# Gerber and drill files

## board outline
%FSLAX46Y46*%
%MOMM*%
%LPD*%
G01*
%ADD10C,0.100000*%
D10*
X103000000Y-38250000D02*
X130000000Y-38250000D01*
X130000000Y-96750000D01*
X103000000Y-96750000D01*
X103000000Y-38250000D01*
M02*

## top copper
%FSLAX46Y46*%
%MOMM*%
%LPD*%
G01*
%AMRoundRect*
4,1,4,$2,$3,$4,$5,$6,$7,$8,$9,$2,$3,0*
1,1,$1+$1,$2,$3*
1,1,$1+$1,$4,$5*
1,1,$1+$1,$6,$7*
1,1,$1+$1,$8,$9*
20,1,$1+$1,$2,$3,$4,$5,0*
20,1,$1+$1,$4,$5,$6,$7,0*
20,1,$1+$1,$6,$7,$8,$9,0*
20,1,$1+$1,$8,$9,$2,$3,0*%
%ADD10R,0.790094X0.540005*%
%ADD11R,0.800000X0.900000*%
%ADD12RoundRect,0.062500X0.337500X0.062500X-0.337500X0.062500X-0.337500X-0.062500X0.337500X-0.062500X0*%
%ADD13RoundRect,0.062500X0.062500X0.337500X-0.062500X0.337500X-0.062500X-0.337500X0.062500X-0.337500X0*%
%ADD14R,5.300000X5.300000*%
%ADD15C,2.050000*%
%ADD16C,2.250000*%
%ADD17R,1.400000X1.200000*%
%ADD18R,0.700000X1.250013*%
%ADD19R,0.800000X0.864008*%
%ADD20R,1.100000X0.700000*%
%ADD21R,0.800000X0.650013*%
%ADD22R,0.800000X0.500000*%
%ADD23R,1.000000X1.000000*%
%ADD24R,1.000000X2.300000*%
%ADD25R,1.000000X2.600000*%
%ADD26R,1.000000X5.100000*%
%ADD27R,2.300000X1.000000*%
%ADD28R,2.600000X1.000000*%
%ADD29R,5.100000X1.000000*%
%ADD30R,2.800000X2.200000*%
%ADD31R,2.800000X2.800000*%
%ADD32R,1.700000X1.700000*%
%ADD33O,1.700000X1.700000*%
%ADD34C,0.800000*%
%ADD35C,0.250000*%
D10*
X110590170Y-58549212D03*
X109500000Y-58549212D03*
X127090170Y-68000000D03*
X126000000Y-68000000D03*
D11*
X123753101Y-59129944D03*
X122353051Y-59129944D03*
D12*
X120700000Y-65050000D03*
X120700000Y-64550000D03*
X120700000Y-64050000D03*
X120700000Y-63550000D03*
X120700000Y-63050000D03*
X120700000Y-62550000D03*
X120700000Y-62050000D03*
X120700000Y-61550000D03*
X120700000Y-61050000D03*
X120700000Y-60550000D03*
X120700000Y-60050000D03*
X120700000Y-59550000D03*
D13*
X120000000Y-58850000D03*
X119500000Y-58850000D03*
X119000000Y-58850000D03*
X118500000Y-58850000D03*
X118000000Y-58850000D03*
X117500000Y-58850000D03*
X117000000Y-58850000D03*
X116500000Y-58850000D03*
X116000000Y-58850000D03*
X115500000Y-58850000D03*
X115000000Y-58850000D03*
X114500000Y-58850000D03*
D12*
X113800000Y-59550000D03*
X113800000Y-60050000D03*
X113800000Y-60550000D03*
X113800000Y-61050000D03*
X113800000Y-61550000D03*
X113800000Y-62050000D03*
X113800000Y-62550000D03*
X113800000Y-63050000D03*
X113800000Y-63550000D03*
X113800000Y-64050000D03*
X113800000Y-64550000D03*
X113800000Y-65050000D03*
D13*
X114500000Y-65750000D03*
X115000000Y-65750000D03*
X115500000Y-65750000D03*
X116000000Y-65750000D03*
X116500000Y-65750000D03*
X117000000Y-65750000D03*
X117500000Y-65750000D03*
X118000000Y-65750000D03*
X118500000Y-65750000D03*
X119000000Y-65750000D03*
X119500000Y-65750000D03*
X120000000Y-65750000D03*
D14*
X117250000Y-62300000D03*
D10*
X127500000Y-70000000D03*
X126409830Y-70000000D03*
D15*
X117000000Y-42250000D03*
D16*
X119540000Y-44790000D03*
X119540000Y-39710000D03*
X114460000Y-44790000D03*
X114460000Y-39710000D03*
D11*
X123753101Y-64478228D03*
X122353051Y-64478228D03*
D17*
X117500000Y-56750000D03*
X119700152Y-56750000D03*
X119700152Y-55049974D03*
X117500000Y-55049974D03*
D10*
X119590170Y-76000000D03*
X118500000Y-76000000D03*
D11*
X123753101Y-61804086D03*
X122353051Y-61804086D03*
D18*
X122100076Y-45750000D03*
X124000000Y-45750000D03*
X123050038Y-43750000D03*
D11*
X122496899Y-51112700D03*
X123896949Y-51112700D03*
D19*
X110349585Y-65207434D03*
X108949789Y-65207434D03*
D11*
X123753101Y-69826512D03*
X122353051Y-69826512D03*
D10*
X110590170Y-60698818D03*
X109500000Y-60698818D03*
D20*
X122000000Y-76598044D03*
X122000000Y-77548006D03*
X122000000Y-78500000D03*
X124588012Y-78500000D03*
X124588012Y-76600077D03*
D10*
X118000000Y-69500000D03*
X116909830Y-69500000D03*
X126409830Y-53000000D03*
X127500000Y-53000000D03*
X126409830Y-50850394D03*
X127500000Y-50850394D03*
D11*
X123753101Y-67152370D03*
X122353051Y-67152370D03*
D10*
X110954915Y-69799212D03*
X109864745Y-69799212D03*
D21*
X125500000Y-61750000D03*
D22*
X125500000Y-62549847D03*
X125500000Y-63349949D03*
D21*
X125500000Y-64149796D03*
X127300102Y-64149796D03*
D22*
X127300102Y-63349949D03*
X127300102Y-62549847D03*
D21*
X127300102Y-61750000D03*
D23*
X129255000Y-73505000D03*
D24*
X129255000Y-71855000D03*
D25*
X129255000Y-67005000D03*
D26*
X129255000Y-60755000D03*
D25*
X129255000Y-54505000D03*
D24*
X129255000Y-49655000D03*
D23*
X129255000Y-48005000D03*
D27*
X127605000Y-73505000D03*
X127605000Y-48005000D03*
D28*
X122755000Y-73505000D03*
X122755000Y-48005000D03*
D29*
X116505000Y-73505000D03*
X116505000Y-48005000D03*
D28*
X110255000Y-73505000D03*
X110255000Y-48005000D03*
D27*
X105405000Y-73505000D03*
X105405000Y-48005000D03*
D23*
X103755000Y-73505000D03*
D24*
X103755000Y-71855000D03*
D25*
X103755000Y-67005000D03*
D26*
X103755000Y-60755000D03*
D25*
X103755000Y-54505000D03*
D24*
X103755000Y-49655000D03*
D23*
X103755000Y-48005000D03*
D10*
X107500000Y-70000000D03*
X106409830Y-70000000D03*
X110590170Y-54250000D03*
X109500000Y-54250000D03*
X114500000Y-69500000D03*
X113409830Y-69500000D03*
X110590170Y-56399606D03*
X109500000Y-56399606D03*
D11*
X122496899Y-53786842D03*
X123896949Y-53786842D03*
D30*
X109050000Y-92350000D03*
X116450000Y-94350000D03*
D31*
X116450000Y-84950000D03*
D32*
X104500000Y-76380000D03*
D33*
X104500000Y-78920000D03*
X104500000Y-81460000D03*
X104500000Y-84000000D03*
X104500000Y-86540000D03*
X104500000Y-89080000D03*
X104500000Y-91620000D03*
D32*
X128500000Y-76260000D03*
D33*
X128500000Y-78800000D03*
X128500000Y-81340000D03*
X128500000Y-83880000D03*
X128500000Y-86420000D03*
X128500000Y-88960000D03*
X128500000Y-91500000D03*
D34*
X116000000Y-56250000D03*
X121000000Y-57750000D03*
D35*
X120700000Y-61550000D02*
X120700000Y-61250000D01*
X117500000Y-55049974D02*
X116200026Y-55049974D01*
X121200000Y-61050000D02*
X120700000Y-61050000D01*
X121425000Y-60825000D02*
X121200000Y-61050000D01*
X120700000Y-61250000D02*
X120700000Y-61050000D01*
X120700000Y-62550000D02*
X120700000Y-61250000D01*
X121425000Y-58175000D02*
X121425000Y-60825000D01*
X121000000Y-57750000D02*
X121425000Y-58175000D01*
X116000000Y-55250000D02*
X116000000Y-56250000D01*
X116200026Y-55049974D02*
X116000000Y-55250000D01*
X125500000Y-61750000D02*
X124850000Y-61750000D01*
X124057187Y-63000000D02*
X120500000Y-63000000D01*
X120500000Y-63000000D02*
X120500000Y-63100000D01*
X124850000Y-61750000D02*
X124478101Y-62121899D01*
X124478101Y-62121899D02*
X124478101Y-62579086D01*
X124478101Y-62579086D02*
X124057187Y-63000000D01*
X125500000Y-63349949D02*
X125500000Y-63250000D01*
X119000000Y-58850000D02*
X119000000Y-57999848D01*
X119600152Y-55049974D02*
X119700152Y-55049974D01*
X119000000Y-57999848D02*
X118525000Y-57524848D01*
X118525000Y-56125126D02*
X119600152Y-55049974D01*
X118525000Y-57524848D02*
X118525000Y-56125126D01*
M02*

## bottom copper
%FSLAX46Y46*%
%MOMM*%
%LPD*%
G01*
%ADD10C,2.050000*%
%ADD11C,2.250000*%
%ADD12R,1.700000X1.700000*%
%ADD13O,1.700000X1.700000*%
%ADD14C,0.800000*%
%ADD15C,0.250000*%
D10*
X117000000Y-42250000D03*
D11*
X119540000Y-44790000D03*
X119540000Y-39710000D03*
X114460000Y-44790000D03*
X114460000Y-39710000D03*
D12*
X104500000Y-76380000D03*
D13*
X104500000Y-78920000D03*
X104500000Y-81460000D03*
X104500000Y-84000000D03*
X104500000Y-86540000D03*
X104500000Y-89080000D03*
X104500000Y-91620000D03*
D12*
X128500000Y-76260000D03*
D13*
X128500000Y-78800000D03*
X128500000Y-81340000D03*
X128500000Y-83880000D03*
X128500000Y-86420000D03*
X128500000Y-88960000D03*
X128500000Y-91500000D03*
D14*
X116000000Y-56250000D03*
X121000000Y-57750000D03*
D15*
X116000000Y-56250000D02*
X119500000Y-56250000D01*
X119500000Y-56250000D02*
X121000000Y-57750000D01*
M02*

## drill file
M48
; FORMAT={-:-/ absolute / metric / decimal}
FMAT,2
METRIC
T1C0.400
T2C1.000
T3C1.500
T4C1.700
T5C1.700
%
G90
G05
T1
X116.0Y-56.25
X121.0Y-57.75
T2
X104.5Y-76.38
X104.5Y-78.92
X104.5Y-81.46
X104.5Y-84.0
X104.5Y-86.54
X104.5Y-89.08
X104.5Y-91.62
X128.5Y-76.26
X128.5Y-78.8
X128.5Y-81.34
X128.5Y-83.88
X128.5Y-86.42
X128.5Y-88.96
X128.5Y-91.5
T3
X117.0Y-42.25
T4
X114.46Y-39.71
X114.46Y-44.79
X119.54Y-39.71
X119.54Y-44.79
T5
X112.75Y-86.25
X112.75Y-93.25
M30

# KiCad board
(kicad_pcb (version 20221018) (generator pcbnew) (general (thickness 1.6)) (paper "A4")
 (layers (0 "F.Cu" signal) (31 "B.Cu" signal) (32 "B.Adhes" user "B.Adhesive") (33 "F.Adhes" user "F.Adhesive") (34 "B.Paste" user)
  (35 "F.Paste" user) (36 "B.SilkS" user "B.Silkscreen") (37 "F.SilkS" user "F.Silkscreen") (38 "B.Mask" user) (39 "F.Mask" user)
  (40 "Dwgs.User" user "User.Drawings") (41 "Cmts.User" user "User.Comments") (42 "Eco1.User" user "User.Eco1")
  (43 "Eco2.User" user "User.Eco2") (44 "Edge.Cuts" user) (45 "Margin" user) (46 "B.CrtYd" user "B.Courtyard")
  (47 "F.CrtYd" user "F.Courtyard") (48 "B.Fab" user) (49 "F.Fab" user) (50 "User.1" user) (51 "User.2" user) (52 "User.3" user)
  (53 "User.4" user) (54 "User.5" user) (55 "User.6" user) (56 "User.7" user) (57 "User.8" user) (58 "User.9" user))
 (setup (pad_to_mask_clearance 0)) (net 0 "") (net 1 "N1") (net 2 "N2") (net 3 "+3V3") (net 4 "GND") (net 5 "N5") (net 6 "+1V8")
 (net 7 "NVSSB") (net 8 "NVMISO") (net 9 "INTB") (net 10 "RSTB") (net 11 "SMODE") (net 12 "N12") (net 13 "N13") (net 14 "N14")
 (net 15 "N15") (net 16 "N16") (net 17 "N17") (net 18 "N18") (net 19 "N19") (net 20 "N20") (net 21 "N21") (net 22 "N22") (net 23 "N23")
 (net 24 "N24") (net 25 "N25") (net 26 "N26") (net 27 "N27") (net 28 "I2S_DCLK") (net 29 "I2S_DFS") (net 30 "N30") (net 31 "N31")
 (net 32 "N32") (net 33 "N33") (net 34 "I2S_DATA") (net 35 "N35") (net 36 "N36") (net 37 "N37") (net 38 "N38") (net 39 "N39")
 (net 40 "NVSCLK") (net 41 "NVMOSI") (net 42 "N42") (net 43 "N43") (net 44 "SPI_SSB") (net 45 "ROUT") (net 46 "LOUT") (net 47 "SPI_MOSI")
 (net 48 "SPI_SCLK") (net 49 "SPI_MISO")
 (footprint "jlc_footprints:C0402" (layer "F.Cu") (at 110.045085 58.549212 180)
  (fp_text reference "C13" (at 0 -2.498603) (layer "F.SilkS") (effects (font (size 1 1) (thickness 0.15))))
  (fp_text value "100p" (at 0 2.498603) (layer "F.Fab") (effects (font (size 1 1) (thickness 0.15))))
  (pad "1" smd rect (at -0.545085 0 180) (size 0.790094 0.540005) (layers "F.Cu" "F.Paste" "F.Mask") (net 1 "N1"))
  (pad "2" smd rect (at 0.545085 0 180) (size 0.790094 0.540005) (layers "F.Cu" "F.Paste" "F.Mask") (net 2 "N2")))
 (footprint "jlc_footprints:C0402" (layer "F.Cu") (at 126.545085 68 180)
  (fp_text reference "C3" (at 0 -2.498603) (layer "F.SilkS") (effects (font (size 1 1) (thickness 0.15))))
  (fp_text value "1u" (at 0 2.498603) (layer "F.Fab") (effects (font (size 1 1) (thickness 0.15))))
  (pad "1" smd rect (at -0.545085 0 180) (size 0.790094 0.540005) (layers "F.Cu" "F.Paste" "F.Mask") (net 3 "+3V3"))
  (pad "2" smd rect (at 0.545085 0 180) (size 0.790094 0.540005) (layers "F.Cu" "F.Paste" "F.Mask") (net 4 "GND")))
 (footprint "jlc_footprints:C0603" (layer "F.Cu") (at 123.053076 59.129944 180)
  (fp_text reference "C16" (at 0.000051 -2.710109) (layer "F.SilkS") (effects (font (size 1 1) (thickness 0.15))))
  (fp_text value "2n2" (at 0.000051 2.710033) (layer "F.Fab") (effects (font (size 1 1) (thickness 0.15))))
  (pad "1" smd rect (at -0.700025 0 180) (size 0.8 0.9) (layers "F.Cu" "F.Paste" "F.Mask") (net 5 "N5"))
  (pad "2" smd rect (at 0.700025 0 180) (size 0.8 0.9) (layers "F.Cu" "F.Paste" "F.Mask") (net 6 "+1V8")))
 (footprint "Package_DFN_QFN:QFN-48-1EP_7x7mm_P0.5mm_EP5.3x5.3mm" (layer "F.Cu") (at 117.25 62.3 180)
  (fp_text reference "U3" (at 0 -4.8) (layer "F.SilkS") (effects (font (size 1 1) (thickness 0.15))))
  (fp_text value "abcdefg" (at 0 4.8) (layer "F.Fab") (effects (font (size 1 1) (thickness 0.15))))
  (pad "" smd roundrect (at -1.98 -1.98 180) (size 1.07 1.07) (layers "F.Paste") (roundrect_rratio 0.2336448598))
  (pad "" smd roundrect (at -1.98 -0.66 180) (size 1.07 1.07) (layers "F.Paste") (roundrect_rratio 0.2336448598))
  (pad "" smd roundrect (at -1.98 0.66 180) (size 1.07 1.07) (layers "F.Paste") (roundrect_rratio 0.2336448598))
  (pad "" smd roundrect (at -1.98 1.98 180) (size 1.07 1.07) (layers "F.Paste") (roundrect_rratio 0.2336448598))
  (pad "" smd roundrect (at -0.66 -1.98 180) (size 1.07 1.07) (layers "F.Paste") (roundrect_rratio 0.2336448598))
  (pad "" smd roundrect (at -0.66 -0.66 180) (size 1.07 1.07) (layers "F.Paste") (roundrect_rratio 0.2336448598))
  (pad "" smd roundrect (at -0.66 0.66 180) (size 1.07 1.07) (layers "F.Paste") (roundrect_rratio 0.2336448598))
  (pad "" smd roundrect (at -0.66 1.98 180) (size 1.07 1.07) (layers "F.Paste") (roundrect_rratio 0.2336448598))
  (pad "" smd roundrect (at 0.66 -1.98 180) (size 1.07 1.07) (layers "F.Paste") (roundrect_rratio 0.2336448598))
  (pad "" smd roundrect (at 0.66 -0.66 180) (size 1.07 1.07) (layers "F.Paste") (roundrect_rratio 0.2336448598))
  (pad "" smd roundrect (at 0.66 0.66 180) (size 1.07 1.07) (layers "F.Paste") (roundrect_rratio 0.2336448598))
  (pad "" smd roundrect (at 0.66 1.98 180) (size 1.07 1.07) (layers "F.Paste") (roundrect_rratio 0.2336448598))
  (pad "" smd roundrect (at 1.98 -1.98 180) (size 1.07 1.07) (layers "F.Paste") (roundrect_rratio 0.2336448598))
  (pad "" smd roundrect (at 1.98 -0.66 180) (size 1.07 1.07) (layers "F.Paste") (roundrect_rratio 0.2336448598))
  (pad "" smd roundrect (at 1.98 0.66 180) (size 1.07 1.07) (layers "F.Paste") (roundrect_rratio 0.2336448598))
  (pad "" smd roundrect (at 1.98 1.98 180) (size 1.07 1.07) (layers "F.Paste") (roundrect_rratio 0.2336448598))
  (pad "1" smd roundrect (at -3.45 -2.75 180) (size 0.8 0.25) (layers "F.Cu" "F.Paste" "F.Mask") (roundrect_rratio 0.25) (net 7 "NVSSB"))
  (pad "2" smd roundrect (at -3.45 -2.25 180) (size 0.8 0.25) (layers "F.Cu" "F.Paste" "F.Mask") (roundrect_rratio 0.25) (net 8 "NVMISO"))
  (pad "3" smd roundrect (at -3.45 -1.75 180) (size 0.8 0.25) (layers "F.Cu" "F.Paste" "F.Mask") (roundrect_rratio 0.25) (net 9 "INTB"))
  (pad "4" smd roundrect (at -3.45 -1.25 180) (size 0.8 0.25) (layers "F.Cu" "F.Paste" "F.Mask") (roundrect_rratio 0.25) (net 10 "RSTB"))
  (pad "5" smd roundrect (at -3.45 -0.75 180) (size 0.8 0.25) (layers "F.Cu" "F.Paste" "F.Mask") (roundrect_rratio 0.25) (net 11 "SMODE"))
  (pad "6" smd roundrect (at -3.45 -0.25 180) (size 0.8 0.25) (layers "F.Cu" "F.Paste" "F.Mask") (roundrect_rratio 0.25) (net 4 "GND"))
  (pad "7" smd roundrect (at -3.45 0.25 180) (size 0.8 0.25) (layers "F.Cu" "F.Paste" "F.Mask") (roundrect_rratio 0.25) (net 4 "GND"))
  (pad "8" smd roundrect (at -3.45 0.75 180) (size 0.8 0.25) (layers "F.Cu" "F.Paste" "F.Mask") (roundrect_rratio 0.25) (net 4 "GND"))
  (pad "9" smd roundrect (at -3.45 1.25 180) (size 0.8 0.25) (layers "F.Cu" "F.Paste" "F.Mask") (roundrect_rratio 0.25) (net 4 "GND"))
  (pad "10" smd roundrect (at -3.45 1.75 180) (size 0.8 0.25) (layers "F.Cu" "F.Paste" "F.Mask") (roundrect_rratio 0.25) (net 2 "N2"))
  (pad "11" smd roundrect (at -3.45 2.25 180) (size 0.8 0.25) (layers "F.Cu" "F.Paste" "F.Mask") (roundrect_rratio 0.25) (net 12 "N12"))
  (pad "12" smd roundrect (at -3.45 2.75 180) (size 0.8 0.25) (layers "F.Cu" "F.Paste" "F.Mask") (roundrect_rratio 0.25) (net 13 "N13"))
  (pad "13" smd roundrect (at -2.75 3.45 180) (size 0.25 0.8) (layers "F.Cu" "F.Paste" "F.Mask") (roundrect_rratio 0.25) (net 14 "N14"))
  (pad "14" smd roundrect (at -2.25 3.45 180) (size 0.25 0.8) (layers "F.Cu" "F.Paste" "F.Mask") (roundrect_rratio 0.25) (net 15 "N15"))
  (pad "15" smd roundrect (at -1.75 3.45 180) (size 0.25 0.8) (layers "F.Cu" "F.Paste" "F.Mask") (roundrect_rratio 0.25) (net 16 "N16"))
  (pad "16" smd roundrect (at -1.25 3.45 180) (size 0.25 0.8) (layers "F.Cu" "F.Paste" "F.Mask") (roundrect_rratio 0.25) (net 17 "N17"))
  (pad "17" smd roundrect (at -0.75 3.45 180) (size 0.25 0.8) (layers "F.Cu" "F.Paste" "F.Mask") (roundrect_rratio 0.25) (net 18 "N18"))
  (pad "18" smd roundrect (at -0.25 3.45 180) (size 0.25 0.8) (layers "F.Cu" "F.Paste" "F.Mask") (roundrect_rratio 0.25) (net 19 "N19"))
  (pad "19" smd roundrect (at 0.25 3.45 180) (size 0.25 0.8) (layers "F.Cu" "F.Paste" "F.Mask") (roundrect_rratio 0.25) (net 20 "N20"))
  (pad "20" smd roundrect (at 0.75 3.45 180) (size 0.25 0.8) (layers "F.Cu" "F.Paste" "F.Mask") (roundrect_rratio 0.25) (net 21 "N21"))
  (pad "21" smd roundrect (at 1.25 3.45 180) (size 0.25 0.8) (layers "F.Cu" "F.Paste" "F.Mask") (roundrect_rratio 0.25) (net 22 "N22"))
  (pad "22" smd roundrect (at 1.75 3.45 180) (size 0.25 0.8) (layers "F.Cu" "F.Paste" "F.Mask") (roundrect_rratio 0.25) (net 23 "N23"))
  (pad "23" smd roundrect (at 2.25 3.45 180) (size 0.25 0.8) (layers "F.Cu" "F.Paste" "F.Mask") (roundrect_rratio 0.25) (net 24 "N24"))
  (pad "24" smd roundrect (at 2.75 3.45 180) (size 0.25 0.8) (layers "F.Cu" "F.Paste" "F.Mask") (roundrect_rratio 0.25) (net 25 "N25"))
  (pad "25" smd roundrect (at 3.45 2.75 180) (size 0.8 0.25) (layers "F.Cu" "F.Paste" "F.Mask") (roundrect_rratio 0.25) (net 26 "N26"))
  (pad "26" smd roundrect (at 3.45 2.25 180) (size 0.8 0.25) (layers "F.Cu" "F.Paste" "F.Mask") (roundrect_rratio 0.25) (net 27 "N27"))
  (pad "27" smd roundrect (at 3.45 1.75 180) (size 0.8 0.25) (layers "F.Cu" "F.Paste" "F.Mask") (roundrect_rratio 0.25) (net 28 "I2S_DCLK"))
  (pad "28" smd roundrect (at 3.45 1.25 180) (size 0.8 0.25) (layers "F.Cu" "F.Paste" "F.Mask") (roundrect_rratio 0.25) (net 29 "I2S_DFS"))
  (pad "29" smd roundrect (at 3.45 0.75 180) (size 0.8 0.25) (layers "F.Cu" "F.Paste" "F.Mask") (roundrect_rratio 0.25) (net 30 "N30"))
  (pad "30" smd roundrect (at 3.45 0.25 180) (size 0.8 0.25) (layers "F.Cu" "F.Paste" "F.Mask") (roundrect_rratio 0.25) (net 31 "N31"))
  (pad "31" smd roundrect (at 3.45 -0.25 180) (size 0.8 0.25) (layers "F.Cu" "F.Paste" "F.Mask") (roundrect_rratio 0.25) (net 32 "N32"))
  (pad "32" smd roundrect (at 3.45 -0.75 180) (size 0.8 0.25) (layers "F.Cu" "F.Paste" "F.Mask") (roundrect_rratio 0.25) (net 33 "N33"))
  (pad "33" smd roundrect (at 3.45 -1.25 180) (size 0.8 0.25) (layers "F.Cu" "F.Paste" "F.Mask") (roundrect_rratio 0.25) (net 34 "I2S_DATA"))
  (pad "34" smd roundrect (at 3.45 -1.75 180) (size 0.8 0.25) (layers "F.Cu" "F.Paste" "F.Mask") (roundrect_rratio 0.25) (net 3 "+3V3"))
  (pad "35" smd roundrect (at 3.45 -2.25 180) (size 0.8 0.25) (layers "F.Cu" "F.Paste" "F.Mask") (roundrect_rratio 0.25) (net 6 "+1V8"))
  (pad "36" smd roundrect (at 3.45 -2.75 180) (size 0.8 0.25) (layers "F.Cu" "F.Paste" "F.Mask") (roundrect_rratio 0.25) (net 5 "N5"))
  (pad "37" smd roundrect (at 2.75 -3.45 180) (size 0.25 0.8) (layers "F.Cu" "F.Paste" "F.Mask") (roundrect_rratio 0.25) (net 6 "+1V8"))
  (pad "38" smd roundrect (at 2.25 -3.45 180) (size 0.25 0.8) (layers "F.Cu" "F.Paste" "F.Mask") (roundrect_rratio 0.25) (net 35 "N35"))
  (pad "39" smd roundrect (at 1.75 -3.45 180) (size 0.25 0.8) (layers "F.Cu" "F.Paste" "F.Mask") (roundrect_rratio 0.25) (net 4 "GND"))
  (pad "40" smd roundrect (at 1.25 -3.45 180) (size 0.25 0.8) (layers "F.Cu" "F.Paste" "F.Mask") (roundrect_rratio 0.25) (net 4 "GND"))
  (pad "41" smd roundrect (at 0.75 -3.45 180) (size 0.25 0.8) (layers "F.Cu" "F.Paste" "F.Mask") (roundrect_rratio 0.25) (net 4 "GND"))
  (pad "42" smd roundrect (at 0.25 -3.45 180) (size 0.25 0.8) (layers "F.Cu" "F.Paste" "F.Mask") (roundrect_rratio 0.25) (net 4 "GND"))
  (pad "43" smd roundrect (at -0.25 -3.45 180) (size 0.25 0.8) (layers "F.Cu" "F.Paste" "F.Mask") (roundrect_rratio 0.25) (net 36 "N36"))
  (pad "44" smd roundrect (at -0.75 -3.45 180) (size 0.25 0.8) (layers "F.Cu" "F.Paste" "F.Mask") (roundrect_rratio 0.25) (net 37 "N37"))
  (pad "45" smd roundrect (at -1.25 -3.45 180) (size 0.25 0.8) (layers "F.Cu" "F.Paste" "F.Mask") (roundrect_rratio 0.25) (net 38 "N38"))
  (pad "46" smd roundrect (at -1.75 -3.45 180) (size 0.25 0.8) (layers "F.Cu" "F.Paste" "F.Mask") (roundrect_rratio 0.25) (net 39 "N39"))
  (pad "47" smd roundrect (at -2.25 -3.45 180) (size 0.25 0.8) (layers "F.Cu" "F.Paste" "F.Mask") (roundrect_rratio 0.25) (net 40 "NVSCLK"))
  (pad "48" smd roundrect (at -2.75 -3.45 180) (size 0.25 0.8) (layers "F.Cu" "F.Paste" "F.Mask") (roundrect_rratio 0.25) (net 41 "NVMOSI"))
  (pad "49" smd rect (at 0 0 180) (size 5.3 5.3) (layers "F.Cu" "F.Mask")))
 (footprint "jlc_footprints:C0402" (layer "F.Cu") (at 126.954915 70 180)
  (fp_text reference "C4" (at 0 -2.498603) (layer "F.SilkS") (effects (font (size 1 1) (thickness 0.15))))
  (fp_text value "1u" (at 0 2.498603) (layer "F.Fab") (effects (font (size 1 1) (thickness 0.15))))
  (pad "1" smd rect (at -0.545085 0 180) (size 0.790094 0.540005) (layers "F.Cu" "F.Paste" "F.Mask") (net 6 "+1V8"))
  (pad "2" smd rect (at 0.545085 0 180) (size 0.790094 0.540005) (layers "F.Cu" "F.Paste" "F.Mask") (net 4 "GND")))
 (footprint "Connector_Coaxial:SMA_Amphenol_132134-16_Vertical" (layer "F.Cu") (at 117 42.25 180)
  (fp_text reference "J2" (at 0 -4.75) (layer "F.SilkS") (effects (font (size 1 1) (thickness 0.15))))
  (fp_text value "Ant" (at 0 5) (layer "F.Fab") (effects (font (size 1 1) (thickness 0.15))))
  (pad "1" thru_hole circle (at 0 0 180) (size 2.05 2.05) (drill 1.5) (layers "*.Cu" "*.Mask") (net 1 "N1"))
  (pad "2" thru_hole circle (at -2.54 -2.54 180) (size 2.25 2.25) (drill 1.7) (layers "*.Cu" "*.Mask") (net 4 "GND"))
  (pad "2" thru_hole circle (at -2.54 2.54 180) (size 2.25 2.25) (drill 1.7) (layers "*.Cu" "*.Mask") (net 4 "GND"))
  (pad "2" thru_hole circle (at 2.54 -2.54 180) (size 2.25 2.25) (drill 1.7) (layers "*.Cu" "*.Mask") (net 4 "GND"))
  (pad "2" thru_hole circle (at 2.54 2.54 180) (size 2.25 2.25) (drill 1.7) (layers "*.Cu" "*.Mask") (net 4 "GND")))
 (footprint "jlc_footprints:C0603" (layer "F.Cu") (at 123.053076 64.478228 180)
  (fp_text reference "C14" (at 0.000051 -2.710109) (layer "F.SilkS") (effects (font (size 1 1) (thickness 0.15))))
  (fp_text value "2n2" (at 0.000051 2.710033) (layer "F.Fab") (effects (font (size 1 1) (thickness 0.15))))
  (pad "1" smd rect (at -0.700025 0 180) (size 0.8 0.9) (layers "F.Cu" "F.Paste" "F.Mask") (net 14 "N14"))
  (pad "2" smd rect (at 0.700025 0 180) (size 0.8 0.9) (layers "F.Cu" "F.Paste" "F.Mask") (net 13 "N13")))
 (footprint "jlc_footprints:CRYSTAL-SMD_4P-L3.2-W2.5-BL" (layer "F.Cu") (at 118.600076 55.899987)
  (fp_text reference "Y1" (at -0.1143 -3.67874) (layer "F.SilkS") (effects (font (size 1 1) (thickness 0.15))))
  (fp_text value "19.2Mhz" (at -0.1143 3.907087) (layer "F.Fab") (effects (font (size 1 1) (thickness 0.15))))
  (pad "1" smd rect (at -1.100076 0.850013) (size 1.4 1.2) (layers "F.Cu" "F.Paste" "F.Mask") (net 17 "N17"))
  (pad "2" smd rect (at 1.100076 0.850013) (size 1.4 1.2) (layers "F.Cu" "F.Paste" "F.Mask") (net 4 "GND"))
  (pad "3" smd rect (at 1.100076 -0.850013) (size 1.4 1.2) (layers "F.Cu" "F.Paste" "F.Mask") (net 16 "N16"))
  (pad "4" smd rect (at -1.100076 -0.850013) (size 1.4 1.2) (layers "F.Cu" "F.Paste" "F.Mask") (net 4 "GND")))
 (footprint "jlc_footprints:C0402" (layer "F.Cu") (at 119.045085 76 180)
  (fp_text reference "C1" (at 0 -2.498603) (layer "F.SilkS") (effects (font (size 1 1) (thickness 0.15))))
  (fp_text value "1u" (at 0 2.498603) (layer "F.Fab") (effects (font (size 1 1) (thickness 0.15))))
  (pad "1" smd rect (at -0.545085 0 180) (size 0.790094 0.540005) (layers "F.Cu" "F.Paste" "F.Mask") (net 4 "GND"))
  (pad "2" smd rect (at 0.545085 0 180) (size 0.790094 0.540005) (layers "F.Cu" "F.Paste" "F.Mask") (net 18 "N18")))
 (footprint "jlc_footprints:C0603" (layer "F.Cu") (at 123.053076 61.804086 180)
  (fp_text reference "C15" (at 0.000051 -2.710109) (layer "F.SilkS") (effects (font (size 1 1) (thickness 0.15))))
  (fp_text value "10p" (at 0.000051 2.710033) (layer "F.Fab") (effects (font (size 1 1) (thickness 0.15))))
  (pad "1" smd rect (at -0.700025 0 180) (size 0.8 0.9) (layers "F.Cu" "F.Paste" "F.Mask") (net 14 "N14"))
  (pad "2" smd rect (at 0.700025 0 180) (size 0.8 0.9) (layers "F.Cu" "F.Paste" "F.Mask") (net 13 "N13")))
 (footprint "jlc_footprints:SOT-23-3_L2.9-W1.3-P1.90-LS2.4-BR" (layer "F.Cu") (at 123.050038 44.75 -90)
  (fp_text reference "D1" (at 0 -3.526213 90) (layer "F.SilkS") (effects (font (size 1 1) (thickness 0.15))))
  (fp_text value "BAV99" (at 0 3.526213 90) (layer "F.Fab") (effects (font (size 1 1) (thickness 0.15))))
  (pad "1" smd rect (at 1 0.949962 270) (size 1.250013 0.7) (layers "F.Cu" "F.Paste" "F.Mask") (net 4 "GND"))
  (pad "2" smd rect (at 1 -0.949962 270) (size 1.250013 0.7) (layers "F.Cu" "F.Paste" "F.Mask") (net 4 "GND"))
  (pad "3" smd rect (at -1 0 270) (size 1.250013 0.7) (layers "F.Cu" "F.Paste" "F.Mask") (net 1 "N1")))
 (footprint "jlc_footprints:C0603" (layer "F.Cu") (at 123.196924 51.1127)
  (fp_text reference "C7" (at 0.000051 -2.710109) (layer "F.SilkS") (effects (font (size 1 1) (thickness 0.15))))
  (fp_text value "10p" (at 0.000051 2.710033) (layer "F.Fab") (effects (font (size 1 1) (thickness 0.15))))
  (pad "1" smd rect (at -0.700025 0) (size 0.8 0.9) (layers "F.Cu" "F.Paste" "F.Mask") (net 4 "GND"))
  (pad "2" smd rect (at 0.700025 0) (size 0.8 0.9) (layers "F.Cu" "F.Paste" "F.Mask") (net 20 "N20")))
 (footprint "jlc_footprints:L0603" (layer "F.Cu") (at 109.649687 65.207434 180)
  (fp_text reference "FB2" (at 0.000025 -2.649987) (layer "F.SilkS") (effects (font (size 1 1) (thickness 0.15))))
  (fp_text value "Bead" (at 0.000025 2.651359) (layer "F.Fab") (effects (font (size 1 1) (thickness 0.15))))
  (pad "1" smd rect (at -0.699898 0) (size 0.8 0.864008) (layers "F.Cu" "F.Paste" "F.Mask") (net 6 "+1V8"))
  (pad "2" smd rect (at 0.699898 0) (size 0.8 0.864008) (layers "F.Cu" "F.Paste" "F.Mask") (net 13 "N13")))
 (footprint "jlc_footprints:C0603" (layer "F.Cu") (at 123.053076 69.826512 180)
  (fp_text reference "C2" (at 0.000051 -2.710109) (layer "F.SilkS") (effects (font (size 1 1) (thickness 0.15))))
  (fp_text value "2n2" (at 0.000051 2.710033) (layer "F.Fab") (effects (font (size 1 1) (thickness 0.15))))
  (pad "1" smd rect (at -0.700025 0 180) (size 0.8 0.9) (layers "F.Cu" "F.Paste" "F.Mask") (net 5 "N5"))
  (pad "2" smd rect (at 0.700025 0 180) (size 0.8 0.9) (layers "F.Cu" "F.Paste" "F.Mask") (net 3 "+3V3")))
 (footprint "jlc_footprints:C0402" (layer "F.Cu") (at 110.045085 60.698818 180)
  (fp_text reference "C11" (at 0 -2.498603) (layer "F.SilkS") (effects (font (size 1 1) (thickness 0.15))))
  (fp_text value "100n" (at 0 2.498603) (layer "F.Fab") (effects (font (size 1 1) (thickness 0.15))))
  (pad "1" smd rect (at -0.545085 0 180) (size 0.790094 0.540005) (layers "F.Cu" "F.Paste" "F.Mask") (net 14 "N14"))
  (pad "2" smd rect (at 0.545085 0 180) (size 0.790094 0.540005) (layers "F.Cu" "F.Paste" "F.Mask") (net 13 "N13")))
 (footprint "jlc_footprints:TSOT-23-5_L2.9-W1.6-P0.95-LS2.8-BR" (layer "F.Cu") (at 123.294006 77.549124 180)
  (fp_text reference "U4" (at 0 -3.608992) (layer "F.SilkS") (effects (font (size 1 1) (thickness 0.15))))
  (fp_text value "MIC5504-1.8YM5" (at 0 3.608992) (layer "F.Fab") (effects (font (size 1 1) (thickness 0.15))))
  (pad "1" smd rect (at 1.294006 0.95108 180) (size 1.1 0.7) (layers "F.Cu" "F.Paste" "F.Mask") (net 3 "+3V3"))
  (pad "2" smd rect (at 1.294006 0.001118 180) (size 1.1 0.7) (layers "F.Cu" "F.Paste" "F.Mask") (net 4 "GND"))
  (pad "3" smd rect (at 1.294006 -0.950876 180) (size 1.1 0.7) (layers "F.Cu" "F.Paste" "F.Mask") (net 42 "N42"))
  (pad "4" smd rect (at -1.294006 -0.950876) (size 1.1 0.7) (layers "F.Cu" "F.Paste" "F.Mask") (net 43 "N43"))
  (pad "5" smd rect (at -1.294006 0.949047) (size 1.1 0.7) (layers "F.Cu" "F.Paste" "F.Mask") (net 6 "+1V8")))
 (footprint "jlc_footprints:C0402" (layer "F.Cu") (at 117.454915 69.5 180)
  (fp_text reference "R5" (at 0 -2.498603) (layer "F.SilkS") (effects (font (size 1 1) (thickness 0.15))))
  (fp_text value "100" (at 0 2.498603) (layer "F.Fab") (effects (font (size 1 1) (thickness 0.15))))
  (pad "1" smd rect (at -0.545085 0 180) (size 0.790094 0.540005) (layers "F.Cu" "F.Paste" "F.Mask") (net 30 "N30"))
  (pad "2" smd rect (at 0.545085 0 180) (size 0.790094 0.540005) (layers "F.Cu" "F.Paste" "F.Mask") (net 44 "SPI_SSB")))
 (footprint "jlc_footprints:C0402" (layer "F.Cu") (at 126.954915 53)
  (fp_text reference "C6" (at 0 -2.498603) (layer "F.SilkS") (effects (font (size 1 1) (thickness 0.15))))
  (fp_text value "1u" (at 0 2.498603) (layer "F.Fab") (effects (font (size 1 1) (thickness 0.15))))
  (pad "1" smd rect (at -0.545085 0) (size 0.790094 0.540005) (layers "F.Cu" "F.Paste" "F.Mask") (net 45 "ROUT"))
  (pad "2" smd rect (at 0.545085 0) (size 0.790094 0.540005) (layers "F.Cu" "F.Paste" "F.Mask") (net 20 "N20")))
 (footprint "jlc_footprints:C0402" (layer "F.Cu") (at 126.954915 50.850394)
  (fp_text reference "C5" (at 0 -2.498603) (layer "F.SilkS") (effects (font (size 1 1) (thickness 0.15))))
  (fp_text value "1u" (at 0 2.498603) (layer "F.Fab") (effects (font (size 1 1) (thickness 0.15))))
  (pad "1" smd rect (at -0.545085 0) (size 0.790094 0.540005) (layers "F.Cu" "F.Paste" "F.Mask") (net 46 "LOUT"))
  (pad "2" smd rect (at 0.545085 0) (size 0.790094 0.540005) (layers "F.Cu" "F.Paste" "F.Mask") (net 19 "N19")))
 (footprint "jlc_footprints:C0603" (layer "F.Cu") (at 123.053076 67.15237 180)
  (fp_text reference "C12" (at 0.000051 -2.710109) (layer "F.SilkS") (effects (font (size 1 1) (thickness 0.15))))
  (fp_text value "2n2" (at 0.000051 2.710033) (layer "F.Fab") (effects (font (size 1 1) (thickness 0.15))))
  (pad "1" smd rect (at -0.700025 0 180) (size 0.8 0.9) (layers "F.Cu" "F.Paste" "F.Mask") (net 5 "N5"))
  (pad "2" smd rect (at 0.700025 0 180) (size 0.8 0.9) (layers "F.Cu" "F.Paste" "F.Mask") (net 6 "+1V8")))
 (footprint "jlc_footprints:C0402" (layer "F.Cu") (at 110.40983 69.799212 180)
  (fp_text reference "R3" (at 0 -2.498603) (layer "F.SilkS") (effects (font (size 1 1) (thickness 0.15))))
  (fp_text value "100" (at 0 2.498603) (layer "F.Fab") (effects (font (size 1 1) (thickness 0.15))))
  (pad "1" smd rect (at -0.545085 0 180) (size 0.790094 0.540005) (layers "F.Cu" "F.Paste" "F.Mask") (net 32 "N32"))
  (pad "2" smd rect (at 0.545085 0 180) (size 0.790094 0.540005) (layers "F.Cu" "F.Paste" "F.Mask") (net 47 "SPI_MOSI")))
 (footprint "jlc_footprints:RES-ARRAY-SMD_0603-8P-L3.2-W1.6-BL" (layer "F.Cu") (at 126.400051 62.949898 -90)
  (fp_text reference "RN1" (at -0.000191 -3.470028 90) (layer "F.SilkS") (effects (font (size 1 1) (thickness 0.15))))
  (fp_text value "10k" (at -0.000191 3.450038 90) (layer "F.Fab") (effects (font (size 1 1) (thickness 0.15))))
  (pad "1" smd rect (at -1.199898 0.900051 270) (size 0.650013 0.8) (layers "F.Cu" "F.Paste" "F.Mask") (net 11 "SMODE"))
  (pad "2" smd rect (at -0.400051 0.900051 270) (size 0.5 0.8) (layers "F.Cu" "F.Paste" "F.Mask") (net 10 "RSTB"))
  (pad "3" smd rect (at 0.400051 0.900051 270) (size 0.5 0.8) (layers "F.Cu" "F.Paste" "F.Mask") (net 9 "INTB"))
  (pad "4" smd rect (at 1.199898 0.900051 270) (size 0.650013 0.8) (layers "F.Cu" "F.Paste" "F.Mask") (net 3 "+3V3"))
  (pad "5" smd rect (at 1.199898 -0.900051 270) (size 0.650013 0.8) (layers "F.Cu" "F.Paste" "F.Mask") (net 42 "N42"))
  (pad "6" smd rect (at 0.400051 -0.900051 270) (size 0.5 0.8) (layers "F.Cu" "F.Paste" "F.Mask") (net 3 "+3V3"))
  (pad "7" smd rect (at -0.400051 -0.900051 270) (size 0.5 0.8) (layers "F.Cu" "F.Paste" "F.Mask") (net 3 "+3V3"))
  (pad "8" smd rect (at -1.199898 -0.900051 270) (size 0.650013 0.8) (layers "F.Cu" "F.Paste" "F.Mask") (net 4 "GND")))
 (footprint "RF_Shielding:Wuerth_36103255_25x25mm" (layer "F.Cu") (at 116.505 60.755 180)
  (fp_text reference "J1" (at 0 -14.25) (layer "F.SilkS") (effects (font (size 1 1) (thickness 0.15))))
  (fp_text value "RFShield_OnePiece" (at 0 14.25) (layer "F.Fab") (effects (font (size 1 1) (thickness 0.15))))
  (pad "1" smd rect (at -12.75 -12.75 180) (size 1 1) (layers "F.Cu" "F.Paste" "F.Mask") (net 4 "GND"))
  (pad "1" smd rect (at -12.75 -11.1 180) (size 1 2.3) (layers "F.Cu" "F.Paste" "F.Mask") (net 4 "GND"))
  (pad "1" smd rect (at -12.75 -6.25 180) (size 1 2.6) (layers "F.Cu" "F.Paste" "F.Mask") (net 4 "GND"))
  (pad "1" smd rect (at -12.75 0 180) (size 1 5.1) (layers "F.Cu" "F.Paste" "F.Mask") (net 4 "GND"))
  (pad "1" smd rect (at -12.75 6.25 180) (size 1 2.6) (layers "F.Cu" "F.Paste" "F.Mask") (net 4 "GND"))
  (pad "1" smd rect (at -12.75 11.1 180) (size 1 2.3) (layers "F.Cu" "F.Paste" "F.Mask") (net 4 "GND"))
  (pad "1" smd rect (at -12.75 12.75 180) (size 1 1) (layers "F.Cu" "F.Paste" "F.Mask") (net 4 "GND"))
  (pad "1" smd rect (at -11.1 -12.75 180) (size 2.3 1) (layers "F.Cu" "F.Paste" "F.Mask") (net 4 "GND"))
  (pad "1" smd rect (at -11.1 12.75 180) (size 2.3 1) (layers "F.Cu" "F.Paste" "F.Mask") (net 4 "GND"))
  (pad "1" smd rect (at -6.25 -12.75 180) (size 2.6 1) (layers "F.Cu" "F.Paste" "F.Mask") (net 4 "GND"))
  (pad "1" smd rect (at -6.25 12.75 180) (size 2.6 1) (layers "F.Cu" "F.Paste" "F.Mask") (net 4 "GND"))
  (pad "1" smd rect (at 0 -12.75 180) (size 5.1 1) (layers "F.Cu" "F.Paste" "F.Mask") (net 4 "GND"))
  (pad "1" smd rect (at 0 12.75 180) (size 5.1 1) (layers "F.Cu" "F.Paste" "F.Mask") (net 4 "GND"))
  (pad "1" smd rect (at 6.25 -12.75 180) (size 2.6 1) (layers "F.Cu" "F.Paste" "F.Mask") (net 4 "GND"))
  (pad "1" smd rect (at 6.25 12.75 180) (size 2.6 1) (layers "F.Cu" "F.Paste" "F.Mask") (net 4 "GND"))
  (pad "1" smd rect (at 11.1 -12.75 180) (size 2.3 1) (layers "F.Cu" "F.Paste" "F.Mask") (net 4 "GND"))
  (pad "1" smd rect (at 11.1 12.75 180) (size 2.3 1) (layers "F.Cu" "F.Paste" "F.Mask") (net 4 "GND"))
  (pad "1" smd rect (at 12.75 -12.75 180) (size 1 1) (layers "F.Cu" "F.Paste" "F.Mask") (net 4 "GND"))
  (pad "1" smd rect (at 12.75 -11.1 180) (size 1 2.3) (layers "F.Cu" "F.Paste" "F.Mask") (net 4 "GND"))
  (pad "1" smd rect (at 12.75 -6.25 180) (size 1 2.6) (layers "F.Cu" "F.Paste" "F.Mask") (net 4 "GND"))
  (pad "1" smd rect (at 12.75 0 180) (size 1 5.1) (layers "F.Cu" "F.Paste" "F.Mask") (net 4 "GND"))
  (pad "1" smd rect (at 12.75 6.25 180) (size 1 2.6) (layers "F.Cu" "F.Paste" "F.Mask") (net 4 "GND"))
  (pad "1" smd rect (at 12.75 11.1 180) (size 1 2.3) (layers "F.Cu" "F.Paste" "F.Mask") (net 4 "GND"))
  (pad "1" smd rect (at 12.75 12.75 180) (size 1 1) (layers "F.Cu" "F.Paste" "F.Mask") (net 4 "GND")))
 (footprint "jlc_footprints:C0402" (layer "F.Cu") (at 106.954915 70 180)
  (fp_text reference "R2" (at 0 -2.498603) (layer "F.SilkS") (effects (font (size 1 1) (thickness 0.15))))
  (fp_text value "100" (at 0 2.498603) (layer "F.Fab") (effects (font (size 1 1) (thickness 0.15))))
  (pad "1" smd rect (at -0.545085 0 180) (size 0.790094 0.540005) (layers "F.Cu" "F.Paste" "F.Mask") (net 31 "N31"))
  (pad "2" smd rect (at 0.545085 0 180) (size 0.790094 0.540005) (layers "F.Cu" "F.Paste" "F.Mask") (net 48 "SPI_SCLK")))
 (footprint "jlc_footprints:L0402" (layer "F.Cu") (at 110.045085 54.25 180)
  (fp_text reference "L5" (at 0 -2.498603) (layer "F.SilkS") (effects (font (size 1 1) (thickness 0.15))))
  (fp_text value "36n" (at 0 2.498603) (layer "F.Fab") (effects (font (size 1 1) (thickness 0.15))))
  (pad "1" smd rect (at -0.545085 0 180) (size 0.790094 0.540005) (layers "F.Cu" "F.Paste" "F.Mask") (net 2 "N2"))
  (pad "2" smd rect (at 0.545085 0 180) (size 0.790094 0.540005) (layers "F.Cu" "F.Paste" "F.Mask") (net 12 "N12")))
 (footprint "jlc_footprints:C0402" (layer "F.Cu") (at 113.954915 69.5 180)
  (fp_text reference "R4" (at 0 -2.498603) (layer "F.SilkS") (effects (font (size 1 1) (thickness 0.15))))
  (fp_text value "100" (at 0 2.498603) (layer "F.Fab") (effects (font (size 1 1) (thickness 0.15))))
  (pad "1" smd rect (at -0.545085 0 180) (size 0.790094 0.540005) (layers "F.Cu" "F.Paste" "F.Mask") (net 33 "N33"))
  (pad "2" smd rect (at 0.545085 0 180) (size 0.790094 0.540005) (layers "F.Cu" "F.Paste" "F.Mask") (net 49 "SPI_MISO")))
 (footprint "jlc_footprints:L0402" (layer "F.Cu") (at 110.045085 56.399606 180)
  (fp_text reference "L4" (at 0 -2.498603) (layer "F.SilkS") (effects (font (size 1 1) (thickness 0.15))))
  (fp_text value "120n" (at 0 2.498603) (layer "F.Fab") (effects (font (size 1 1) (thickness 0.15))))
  (pad "1" smd rect (at -0.545085 0 180) (size 0.790094 0.540005) (layers "F.Cu" "F.Paste" "F.Mask") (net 2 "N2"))
  (pad "2" smd rect (at 0.545085 0 180) (size 0.790094 0.540005) (layers "F.Cu" "F.Paste" "F.Mask") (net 4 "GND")))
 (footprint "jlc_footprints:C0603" (layer "F.Cu") (at 123.196924 53.786842)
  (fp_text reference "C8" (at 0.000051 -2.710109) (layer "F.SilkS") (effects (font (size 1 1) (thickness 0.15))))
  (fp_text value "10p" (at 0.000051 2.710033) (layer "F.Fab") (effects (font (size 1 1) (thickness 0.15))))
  (pad "1" smd rect (at -0.700025 0) (size 0.8 0.9) (layers "F.Cu" "F.Paste" "F.Mask") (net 4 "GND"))
  (pad "2" smd rect (at 0.700025 0) (size 0.8 0.9) (layers "F.Cu" "F.Paste" "F.Mask") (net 19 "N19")))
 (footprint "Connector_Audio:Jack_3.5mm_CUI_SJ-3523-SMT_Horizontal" (layer "F.Cu") (at 112.75 90.75 180)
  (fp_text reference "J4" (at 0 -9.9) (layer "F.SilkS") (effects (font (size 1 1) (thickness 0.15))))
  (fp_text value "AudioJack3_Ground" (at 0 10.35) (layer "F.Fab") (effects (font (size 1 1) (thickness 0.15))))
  (pad "" np_thru_hole circle (at 0 -2.5 180) (size 1.7 1.7) (drill 1.7) (layers "*.Cu" "*.Mask"))
  (pad "" np_thru_hole circle (at 0 4.5 180) (size 1.7 1.7) (drill 1.7) (layers "*.Cu" "*.Mask"))
  (pad "R" smd rect (at 3.7 -1.6 180) (size 2.8 2.2) (layers "F.Cu" "F.Paste" "F.Mask") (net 45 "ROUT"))
  (pad "S" smd rect (at -3.7 -3.6 180) (size 2.8 2.2) (layers "F.Cu" "F.Paste" "F.Mask") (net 4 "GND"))
  (pad "T" smd rect (at -3.7 5.8 180) (size 2.8 2.8) (layers "F.Cu" "F.Paste" "F.Mask") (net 46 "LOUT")))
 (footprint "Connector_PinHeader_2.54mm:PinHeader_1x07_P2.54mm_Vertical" (layer "B.Cu") (at 104.5 76.38 180)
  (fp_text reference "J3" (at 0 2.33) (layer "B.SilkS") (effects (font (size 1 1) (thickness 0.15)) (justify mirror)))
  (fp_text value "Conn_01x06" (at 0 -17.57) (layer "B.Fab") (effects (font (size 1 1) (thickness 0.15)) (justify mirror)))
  (pad "1" thru_hole rect (at 0 0 180) (size 1.7 1.7) (drill 1) (layers "*.Cu" "*.Mask") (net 4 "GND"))
  (pad "2" thru_hole oval (at 0 -2.54 180) (size 1.7 1.7) (drill 1) (layers "*.Cu" "*.Mask") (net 3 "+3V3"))
  (pad "3" thru_hole oval (at 0 -5.08 180) (size 1.7 1.7) (drill 1) (layers "*.Cu" "*.Mask") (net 11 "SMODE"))
  (pad "4" thru_hole oval (at 0 -7.62 180) (size 1.7 1.7) (drill 1) (layers "*.Cu" "*.Mask") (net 9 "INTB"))
  (pad "5" thru_hole oval (at 0 -10.16 180) (size 1.7 1.7) (drill 1) (layers "*.Cu" "*.Mask") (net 10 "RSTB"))
  (pad "6" thru_hole oval (at 0 -12.7 180) (size 1.7 1.7) (drill 1) (layers "*.Cu" "*.Mask") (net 46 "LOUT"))
  (pad "7" thru_hole oval (at 0 -15.24 180) (size 1.7 1.7) (drill 1) (layers "*.Cu" "*.Mask") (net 45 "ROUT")))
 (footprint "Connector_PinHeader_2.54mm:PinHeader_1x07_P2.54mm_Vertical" (layer "B.Cu") (at 128.5 76.26 180)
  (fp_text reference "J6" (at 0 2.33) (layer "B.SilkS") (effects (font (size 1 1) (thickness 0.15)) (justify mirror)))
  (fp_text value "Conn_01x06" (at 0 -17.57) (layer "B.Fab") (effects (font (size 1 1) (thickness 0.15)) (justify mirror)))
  (pad "1" thru_hole rect (at 0 0 180) (size 1.7 1.7) (drill 1) (layers "*.Cu" "*.Mask") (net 49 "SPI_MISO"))
  (pad "2" thru_hole oval (at 0 -2.54 180) (size 1.7 1.7) (drill 1) (layers "*.Cu" "*.Mask") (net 47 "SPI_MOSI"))
  (pad "3" thru_hole oval (at 0 -5.08 180) (size 1.7 1.7) (drill 1) (layers "*.Cu" "*.Mask") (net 44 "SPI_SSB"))
  (pad "4" thru_hole oval (at 0 -7.62 180) (size 1.7 1.7) (drill 1) (layers "*.Cu" "*.Mask") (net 48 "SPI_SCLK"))
  (pad "5" thru_hole oval (at 0 -10.16 180) (size 1.7 1.7) (drill 1) (layers "*.Cu" "*.Mask") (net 28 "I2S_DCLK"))
  (pad "6" thru_hole oval (at 0 -12.7 180) (size 1.7 1.7) (drill 1) (layers "*.Cu" "*.Mask") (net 29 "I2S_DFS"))
  (pad "7" thru_hole oval (at 0 -15.24 180) (size 1.7 1.7) (drill 1) (layers "*.Cu" "*.Mask") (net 34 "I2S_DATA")))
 (gr_rect (start 103 38.25) (end 130 96.75) (stroke (width 0.1) (type default)) (fill none) (layer "Edge.Cuts"))
 (segment (start 120.7 61.55) (end 120.7 61.25) (width 0.25) (layer "F.Cu") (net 4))
 (segment (start 117.5 55.049974) (end 116.200026 55.049974) (width 0.25) (layer "F.Cu") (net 4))
 (segment (start 121.2 61.05) (end 120.7 61.05) (width 0.25) (layer "F.Cu") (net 4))
 (segment (start 121.425 60.825) (end 121.2 61.05) (width 0.25) (layer "F.Cu") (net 4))
 (segment (start 120.7 61.25) (end 120.7 61.05) (width 0.25) (layer "F.Cu") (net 4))
 (segment (start 120.7 62.55) (end 120.7 61.25) (width 0.25) (layer "F.Cu") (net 4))
 (segment (start 121.425 58.175) (end 121.425 60.825) (width 0.25) (layer "F.Cu") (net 4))
 (segment (start 121 57.75) (end 121.425 58.175) (width 0.25) (layer "F.Cu") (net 4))
 (segment (start 116 55.25) (end 116 56.25) (width 0.25) (layer "F.Cu") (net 4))
 (segment (start 116.200026 55.049974) (end 116 55.25) (width 0.25) (layer "F.Cu") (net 4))
 (via (at 116 56.25) (size 0.8) (drill 0.4) (layers "F.Cu" "B.Cu") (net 4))
 (via (at 121 57.75) (size 0.8) (drill 0.4) (layers "F.Cu" "B.Cu") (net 4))
 (segment (start 116 56.25) (end 119.5 56.25) (width 0.25) (layer "B.Cu") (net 4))
 (segment (start 119.5 56.25) (end 121 57.75) (width 0.25) (layer "B.Cu") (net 4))
 (segment (start 125.5 61.75) (end 124.85 61.75) (width 0.25) (layer "F.Cu") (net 11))
 (segment (start 124.057187 63) (end 120.5 63) (width 0.25) (layer "F.Cu") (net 11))
 (segment (start 120.5 63) (end 120.5 63.1) (width 0.25) (layer "F.Cu") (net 11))
 (segment (start 124.85 61.75) (end 124.478101 62.121899) (width 0.25) (layer "F.Cu") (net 11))
 (segment (start 124.478101 62.121899) (end 124.478101 62.579086) (width 0.25) (layer "F.Cu") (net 11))
 (segment (start 124.478101 62.579086) (end 124.057187 63) (width 0.25) (layer "F.Cu") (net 11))
 (segment (start 125.5 63.349949) (end 125.5 63.25) (width 0.25) (layer "F.Cu") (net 9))
 (segment (start 119 58.85) (end 119 57.999848) (width 0.25) (layer "F.Cu") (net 16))
 (segment (start 119.600152 55.049974) (end 119.700152 55.049974) (width 0.25) (layer "F.Cu") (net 16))
 (segment (start 119 57.999848) (end 118.525 57.524848) (width 0.25) (layer "F.Cu") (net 16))
 (segment (start 118.525 56.125126) (end 119.600152 55.049974) (width 0.25) (layer "F.Cu") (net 16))
 (segment (start 118.525 57.524848) (end 118.525 56.125126) (width 0.25) (layer "F.Cu") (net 16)))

